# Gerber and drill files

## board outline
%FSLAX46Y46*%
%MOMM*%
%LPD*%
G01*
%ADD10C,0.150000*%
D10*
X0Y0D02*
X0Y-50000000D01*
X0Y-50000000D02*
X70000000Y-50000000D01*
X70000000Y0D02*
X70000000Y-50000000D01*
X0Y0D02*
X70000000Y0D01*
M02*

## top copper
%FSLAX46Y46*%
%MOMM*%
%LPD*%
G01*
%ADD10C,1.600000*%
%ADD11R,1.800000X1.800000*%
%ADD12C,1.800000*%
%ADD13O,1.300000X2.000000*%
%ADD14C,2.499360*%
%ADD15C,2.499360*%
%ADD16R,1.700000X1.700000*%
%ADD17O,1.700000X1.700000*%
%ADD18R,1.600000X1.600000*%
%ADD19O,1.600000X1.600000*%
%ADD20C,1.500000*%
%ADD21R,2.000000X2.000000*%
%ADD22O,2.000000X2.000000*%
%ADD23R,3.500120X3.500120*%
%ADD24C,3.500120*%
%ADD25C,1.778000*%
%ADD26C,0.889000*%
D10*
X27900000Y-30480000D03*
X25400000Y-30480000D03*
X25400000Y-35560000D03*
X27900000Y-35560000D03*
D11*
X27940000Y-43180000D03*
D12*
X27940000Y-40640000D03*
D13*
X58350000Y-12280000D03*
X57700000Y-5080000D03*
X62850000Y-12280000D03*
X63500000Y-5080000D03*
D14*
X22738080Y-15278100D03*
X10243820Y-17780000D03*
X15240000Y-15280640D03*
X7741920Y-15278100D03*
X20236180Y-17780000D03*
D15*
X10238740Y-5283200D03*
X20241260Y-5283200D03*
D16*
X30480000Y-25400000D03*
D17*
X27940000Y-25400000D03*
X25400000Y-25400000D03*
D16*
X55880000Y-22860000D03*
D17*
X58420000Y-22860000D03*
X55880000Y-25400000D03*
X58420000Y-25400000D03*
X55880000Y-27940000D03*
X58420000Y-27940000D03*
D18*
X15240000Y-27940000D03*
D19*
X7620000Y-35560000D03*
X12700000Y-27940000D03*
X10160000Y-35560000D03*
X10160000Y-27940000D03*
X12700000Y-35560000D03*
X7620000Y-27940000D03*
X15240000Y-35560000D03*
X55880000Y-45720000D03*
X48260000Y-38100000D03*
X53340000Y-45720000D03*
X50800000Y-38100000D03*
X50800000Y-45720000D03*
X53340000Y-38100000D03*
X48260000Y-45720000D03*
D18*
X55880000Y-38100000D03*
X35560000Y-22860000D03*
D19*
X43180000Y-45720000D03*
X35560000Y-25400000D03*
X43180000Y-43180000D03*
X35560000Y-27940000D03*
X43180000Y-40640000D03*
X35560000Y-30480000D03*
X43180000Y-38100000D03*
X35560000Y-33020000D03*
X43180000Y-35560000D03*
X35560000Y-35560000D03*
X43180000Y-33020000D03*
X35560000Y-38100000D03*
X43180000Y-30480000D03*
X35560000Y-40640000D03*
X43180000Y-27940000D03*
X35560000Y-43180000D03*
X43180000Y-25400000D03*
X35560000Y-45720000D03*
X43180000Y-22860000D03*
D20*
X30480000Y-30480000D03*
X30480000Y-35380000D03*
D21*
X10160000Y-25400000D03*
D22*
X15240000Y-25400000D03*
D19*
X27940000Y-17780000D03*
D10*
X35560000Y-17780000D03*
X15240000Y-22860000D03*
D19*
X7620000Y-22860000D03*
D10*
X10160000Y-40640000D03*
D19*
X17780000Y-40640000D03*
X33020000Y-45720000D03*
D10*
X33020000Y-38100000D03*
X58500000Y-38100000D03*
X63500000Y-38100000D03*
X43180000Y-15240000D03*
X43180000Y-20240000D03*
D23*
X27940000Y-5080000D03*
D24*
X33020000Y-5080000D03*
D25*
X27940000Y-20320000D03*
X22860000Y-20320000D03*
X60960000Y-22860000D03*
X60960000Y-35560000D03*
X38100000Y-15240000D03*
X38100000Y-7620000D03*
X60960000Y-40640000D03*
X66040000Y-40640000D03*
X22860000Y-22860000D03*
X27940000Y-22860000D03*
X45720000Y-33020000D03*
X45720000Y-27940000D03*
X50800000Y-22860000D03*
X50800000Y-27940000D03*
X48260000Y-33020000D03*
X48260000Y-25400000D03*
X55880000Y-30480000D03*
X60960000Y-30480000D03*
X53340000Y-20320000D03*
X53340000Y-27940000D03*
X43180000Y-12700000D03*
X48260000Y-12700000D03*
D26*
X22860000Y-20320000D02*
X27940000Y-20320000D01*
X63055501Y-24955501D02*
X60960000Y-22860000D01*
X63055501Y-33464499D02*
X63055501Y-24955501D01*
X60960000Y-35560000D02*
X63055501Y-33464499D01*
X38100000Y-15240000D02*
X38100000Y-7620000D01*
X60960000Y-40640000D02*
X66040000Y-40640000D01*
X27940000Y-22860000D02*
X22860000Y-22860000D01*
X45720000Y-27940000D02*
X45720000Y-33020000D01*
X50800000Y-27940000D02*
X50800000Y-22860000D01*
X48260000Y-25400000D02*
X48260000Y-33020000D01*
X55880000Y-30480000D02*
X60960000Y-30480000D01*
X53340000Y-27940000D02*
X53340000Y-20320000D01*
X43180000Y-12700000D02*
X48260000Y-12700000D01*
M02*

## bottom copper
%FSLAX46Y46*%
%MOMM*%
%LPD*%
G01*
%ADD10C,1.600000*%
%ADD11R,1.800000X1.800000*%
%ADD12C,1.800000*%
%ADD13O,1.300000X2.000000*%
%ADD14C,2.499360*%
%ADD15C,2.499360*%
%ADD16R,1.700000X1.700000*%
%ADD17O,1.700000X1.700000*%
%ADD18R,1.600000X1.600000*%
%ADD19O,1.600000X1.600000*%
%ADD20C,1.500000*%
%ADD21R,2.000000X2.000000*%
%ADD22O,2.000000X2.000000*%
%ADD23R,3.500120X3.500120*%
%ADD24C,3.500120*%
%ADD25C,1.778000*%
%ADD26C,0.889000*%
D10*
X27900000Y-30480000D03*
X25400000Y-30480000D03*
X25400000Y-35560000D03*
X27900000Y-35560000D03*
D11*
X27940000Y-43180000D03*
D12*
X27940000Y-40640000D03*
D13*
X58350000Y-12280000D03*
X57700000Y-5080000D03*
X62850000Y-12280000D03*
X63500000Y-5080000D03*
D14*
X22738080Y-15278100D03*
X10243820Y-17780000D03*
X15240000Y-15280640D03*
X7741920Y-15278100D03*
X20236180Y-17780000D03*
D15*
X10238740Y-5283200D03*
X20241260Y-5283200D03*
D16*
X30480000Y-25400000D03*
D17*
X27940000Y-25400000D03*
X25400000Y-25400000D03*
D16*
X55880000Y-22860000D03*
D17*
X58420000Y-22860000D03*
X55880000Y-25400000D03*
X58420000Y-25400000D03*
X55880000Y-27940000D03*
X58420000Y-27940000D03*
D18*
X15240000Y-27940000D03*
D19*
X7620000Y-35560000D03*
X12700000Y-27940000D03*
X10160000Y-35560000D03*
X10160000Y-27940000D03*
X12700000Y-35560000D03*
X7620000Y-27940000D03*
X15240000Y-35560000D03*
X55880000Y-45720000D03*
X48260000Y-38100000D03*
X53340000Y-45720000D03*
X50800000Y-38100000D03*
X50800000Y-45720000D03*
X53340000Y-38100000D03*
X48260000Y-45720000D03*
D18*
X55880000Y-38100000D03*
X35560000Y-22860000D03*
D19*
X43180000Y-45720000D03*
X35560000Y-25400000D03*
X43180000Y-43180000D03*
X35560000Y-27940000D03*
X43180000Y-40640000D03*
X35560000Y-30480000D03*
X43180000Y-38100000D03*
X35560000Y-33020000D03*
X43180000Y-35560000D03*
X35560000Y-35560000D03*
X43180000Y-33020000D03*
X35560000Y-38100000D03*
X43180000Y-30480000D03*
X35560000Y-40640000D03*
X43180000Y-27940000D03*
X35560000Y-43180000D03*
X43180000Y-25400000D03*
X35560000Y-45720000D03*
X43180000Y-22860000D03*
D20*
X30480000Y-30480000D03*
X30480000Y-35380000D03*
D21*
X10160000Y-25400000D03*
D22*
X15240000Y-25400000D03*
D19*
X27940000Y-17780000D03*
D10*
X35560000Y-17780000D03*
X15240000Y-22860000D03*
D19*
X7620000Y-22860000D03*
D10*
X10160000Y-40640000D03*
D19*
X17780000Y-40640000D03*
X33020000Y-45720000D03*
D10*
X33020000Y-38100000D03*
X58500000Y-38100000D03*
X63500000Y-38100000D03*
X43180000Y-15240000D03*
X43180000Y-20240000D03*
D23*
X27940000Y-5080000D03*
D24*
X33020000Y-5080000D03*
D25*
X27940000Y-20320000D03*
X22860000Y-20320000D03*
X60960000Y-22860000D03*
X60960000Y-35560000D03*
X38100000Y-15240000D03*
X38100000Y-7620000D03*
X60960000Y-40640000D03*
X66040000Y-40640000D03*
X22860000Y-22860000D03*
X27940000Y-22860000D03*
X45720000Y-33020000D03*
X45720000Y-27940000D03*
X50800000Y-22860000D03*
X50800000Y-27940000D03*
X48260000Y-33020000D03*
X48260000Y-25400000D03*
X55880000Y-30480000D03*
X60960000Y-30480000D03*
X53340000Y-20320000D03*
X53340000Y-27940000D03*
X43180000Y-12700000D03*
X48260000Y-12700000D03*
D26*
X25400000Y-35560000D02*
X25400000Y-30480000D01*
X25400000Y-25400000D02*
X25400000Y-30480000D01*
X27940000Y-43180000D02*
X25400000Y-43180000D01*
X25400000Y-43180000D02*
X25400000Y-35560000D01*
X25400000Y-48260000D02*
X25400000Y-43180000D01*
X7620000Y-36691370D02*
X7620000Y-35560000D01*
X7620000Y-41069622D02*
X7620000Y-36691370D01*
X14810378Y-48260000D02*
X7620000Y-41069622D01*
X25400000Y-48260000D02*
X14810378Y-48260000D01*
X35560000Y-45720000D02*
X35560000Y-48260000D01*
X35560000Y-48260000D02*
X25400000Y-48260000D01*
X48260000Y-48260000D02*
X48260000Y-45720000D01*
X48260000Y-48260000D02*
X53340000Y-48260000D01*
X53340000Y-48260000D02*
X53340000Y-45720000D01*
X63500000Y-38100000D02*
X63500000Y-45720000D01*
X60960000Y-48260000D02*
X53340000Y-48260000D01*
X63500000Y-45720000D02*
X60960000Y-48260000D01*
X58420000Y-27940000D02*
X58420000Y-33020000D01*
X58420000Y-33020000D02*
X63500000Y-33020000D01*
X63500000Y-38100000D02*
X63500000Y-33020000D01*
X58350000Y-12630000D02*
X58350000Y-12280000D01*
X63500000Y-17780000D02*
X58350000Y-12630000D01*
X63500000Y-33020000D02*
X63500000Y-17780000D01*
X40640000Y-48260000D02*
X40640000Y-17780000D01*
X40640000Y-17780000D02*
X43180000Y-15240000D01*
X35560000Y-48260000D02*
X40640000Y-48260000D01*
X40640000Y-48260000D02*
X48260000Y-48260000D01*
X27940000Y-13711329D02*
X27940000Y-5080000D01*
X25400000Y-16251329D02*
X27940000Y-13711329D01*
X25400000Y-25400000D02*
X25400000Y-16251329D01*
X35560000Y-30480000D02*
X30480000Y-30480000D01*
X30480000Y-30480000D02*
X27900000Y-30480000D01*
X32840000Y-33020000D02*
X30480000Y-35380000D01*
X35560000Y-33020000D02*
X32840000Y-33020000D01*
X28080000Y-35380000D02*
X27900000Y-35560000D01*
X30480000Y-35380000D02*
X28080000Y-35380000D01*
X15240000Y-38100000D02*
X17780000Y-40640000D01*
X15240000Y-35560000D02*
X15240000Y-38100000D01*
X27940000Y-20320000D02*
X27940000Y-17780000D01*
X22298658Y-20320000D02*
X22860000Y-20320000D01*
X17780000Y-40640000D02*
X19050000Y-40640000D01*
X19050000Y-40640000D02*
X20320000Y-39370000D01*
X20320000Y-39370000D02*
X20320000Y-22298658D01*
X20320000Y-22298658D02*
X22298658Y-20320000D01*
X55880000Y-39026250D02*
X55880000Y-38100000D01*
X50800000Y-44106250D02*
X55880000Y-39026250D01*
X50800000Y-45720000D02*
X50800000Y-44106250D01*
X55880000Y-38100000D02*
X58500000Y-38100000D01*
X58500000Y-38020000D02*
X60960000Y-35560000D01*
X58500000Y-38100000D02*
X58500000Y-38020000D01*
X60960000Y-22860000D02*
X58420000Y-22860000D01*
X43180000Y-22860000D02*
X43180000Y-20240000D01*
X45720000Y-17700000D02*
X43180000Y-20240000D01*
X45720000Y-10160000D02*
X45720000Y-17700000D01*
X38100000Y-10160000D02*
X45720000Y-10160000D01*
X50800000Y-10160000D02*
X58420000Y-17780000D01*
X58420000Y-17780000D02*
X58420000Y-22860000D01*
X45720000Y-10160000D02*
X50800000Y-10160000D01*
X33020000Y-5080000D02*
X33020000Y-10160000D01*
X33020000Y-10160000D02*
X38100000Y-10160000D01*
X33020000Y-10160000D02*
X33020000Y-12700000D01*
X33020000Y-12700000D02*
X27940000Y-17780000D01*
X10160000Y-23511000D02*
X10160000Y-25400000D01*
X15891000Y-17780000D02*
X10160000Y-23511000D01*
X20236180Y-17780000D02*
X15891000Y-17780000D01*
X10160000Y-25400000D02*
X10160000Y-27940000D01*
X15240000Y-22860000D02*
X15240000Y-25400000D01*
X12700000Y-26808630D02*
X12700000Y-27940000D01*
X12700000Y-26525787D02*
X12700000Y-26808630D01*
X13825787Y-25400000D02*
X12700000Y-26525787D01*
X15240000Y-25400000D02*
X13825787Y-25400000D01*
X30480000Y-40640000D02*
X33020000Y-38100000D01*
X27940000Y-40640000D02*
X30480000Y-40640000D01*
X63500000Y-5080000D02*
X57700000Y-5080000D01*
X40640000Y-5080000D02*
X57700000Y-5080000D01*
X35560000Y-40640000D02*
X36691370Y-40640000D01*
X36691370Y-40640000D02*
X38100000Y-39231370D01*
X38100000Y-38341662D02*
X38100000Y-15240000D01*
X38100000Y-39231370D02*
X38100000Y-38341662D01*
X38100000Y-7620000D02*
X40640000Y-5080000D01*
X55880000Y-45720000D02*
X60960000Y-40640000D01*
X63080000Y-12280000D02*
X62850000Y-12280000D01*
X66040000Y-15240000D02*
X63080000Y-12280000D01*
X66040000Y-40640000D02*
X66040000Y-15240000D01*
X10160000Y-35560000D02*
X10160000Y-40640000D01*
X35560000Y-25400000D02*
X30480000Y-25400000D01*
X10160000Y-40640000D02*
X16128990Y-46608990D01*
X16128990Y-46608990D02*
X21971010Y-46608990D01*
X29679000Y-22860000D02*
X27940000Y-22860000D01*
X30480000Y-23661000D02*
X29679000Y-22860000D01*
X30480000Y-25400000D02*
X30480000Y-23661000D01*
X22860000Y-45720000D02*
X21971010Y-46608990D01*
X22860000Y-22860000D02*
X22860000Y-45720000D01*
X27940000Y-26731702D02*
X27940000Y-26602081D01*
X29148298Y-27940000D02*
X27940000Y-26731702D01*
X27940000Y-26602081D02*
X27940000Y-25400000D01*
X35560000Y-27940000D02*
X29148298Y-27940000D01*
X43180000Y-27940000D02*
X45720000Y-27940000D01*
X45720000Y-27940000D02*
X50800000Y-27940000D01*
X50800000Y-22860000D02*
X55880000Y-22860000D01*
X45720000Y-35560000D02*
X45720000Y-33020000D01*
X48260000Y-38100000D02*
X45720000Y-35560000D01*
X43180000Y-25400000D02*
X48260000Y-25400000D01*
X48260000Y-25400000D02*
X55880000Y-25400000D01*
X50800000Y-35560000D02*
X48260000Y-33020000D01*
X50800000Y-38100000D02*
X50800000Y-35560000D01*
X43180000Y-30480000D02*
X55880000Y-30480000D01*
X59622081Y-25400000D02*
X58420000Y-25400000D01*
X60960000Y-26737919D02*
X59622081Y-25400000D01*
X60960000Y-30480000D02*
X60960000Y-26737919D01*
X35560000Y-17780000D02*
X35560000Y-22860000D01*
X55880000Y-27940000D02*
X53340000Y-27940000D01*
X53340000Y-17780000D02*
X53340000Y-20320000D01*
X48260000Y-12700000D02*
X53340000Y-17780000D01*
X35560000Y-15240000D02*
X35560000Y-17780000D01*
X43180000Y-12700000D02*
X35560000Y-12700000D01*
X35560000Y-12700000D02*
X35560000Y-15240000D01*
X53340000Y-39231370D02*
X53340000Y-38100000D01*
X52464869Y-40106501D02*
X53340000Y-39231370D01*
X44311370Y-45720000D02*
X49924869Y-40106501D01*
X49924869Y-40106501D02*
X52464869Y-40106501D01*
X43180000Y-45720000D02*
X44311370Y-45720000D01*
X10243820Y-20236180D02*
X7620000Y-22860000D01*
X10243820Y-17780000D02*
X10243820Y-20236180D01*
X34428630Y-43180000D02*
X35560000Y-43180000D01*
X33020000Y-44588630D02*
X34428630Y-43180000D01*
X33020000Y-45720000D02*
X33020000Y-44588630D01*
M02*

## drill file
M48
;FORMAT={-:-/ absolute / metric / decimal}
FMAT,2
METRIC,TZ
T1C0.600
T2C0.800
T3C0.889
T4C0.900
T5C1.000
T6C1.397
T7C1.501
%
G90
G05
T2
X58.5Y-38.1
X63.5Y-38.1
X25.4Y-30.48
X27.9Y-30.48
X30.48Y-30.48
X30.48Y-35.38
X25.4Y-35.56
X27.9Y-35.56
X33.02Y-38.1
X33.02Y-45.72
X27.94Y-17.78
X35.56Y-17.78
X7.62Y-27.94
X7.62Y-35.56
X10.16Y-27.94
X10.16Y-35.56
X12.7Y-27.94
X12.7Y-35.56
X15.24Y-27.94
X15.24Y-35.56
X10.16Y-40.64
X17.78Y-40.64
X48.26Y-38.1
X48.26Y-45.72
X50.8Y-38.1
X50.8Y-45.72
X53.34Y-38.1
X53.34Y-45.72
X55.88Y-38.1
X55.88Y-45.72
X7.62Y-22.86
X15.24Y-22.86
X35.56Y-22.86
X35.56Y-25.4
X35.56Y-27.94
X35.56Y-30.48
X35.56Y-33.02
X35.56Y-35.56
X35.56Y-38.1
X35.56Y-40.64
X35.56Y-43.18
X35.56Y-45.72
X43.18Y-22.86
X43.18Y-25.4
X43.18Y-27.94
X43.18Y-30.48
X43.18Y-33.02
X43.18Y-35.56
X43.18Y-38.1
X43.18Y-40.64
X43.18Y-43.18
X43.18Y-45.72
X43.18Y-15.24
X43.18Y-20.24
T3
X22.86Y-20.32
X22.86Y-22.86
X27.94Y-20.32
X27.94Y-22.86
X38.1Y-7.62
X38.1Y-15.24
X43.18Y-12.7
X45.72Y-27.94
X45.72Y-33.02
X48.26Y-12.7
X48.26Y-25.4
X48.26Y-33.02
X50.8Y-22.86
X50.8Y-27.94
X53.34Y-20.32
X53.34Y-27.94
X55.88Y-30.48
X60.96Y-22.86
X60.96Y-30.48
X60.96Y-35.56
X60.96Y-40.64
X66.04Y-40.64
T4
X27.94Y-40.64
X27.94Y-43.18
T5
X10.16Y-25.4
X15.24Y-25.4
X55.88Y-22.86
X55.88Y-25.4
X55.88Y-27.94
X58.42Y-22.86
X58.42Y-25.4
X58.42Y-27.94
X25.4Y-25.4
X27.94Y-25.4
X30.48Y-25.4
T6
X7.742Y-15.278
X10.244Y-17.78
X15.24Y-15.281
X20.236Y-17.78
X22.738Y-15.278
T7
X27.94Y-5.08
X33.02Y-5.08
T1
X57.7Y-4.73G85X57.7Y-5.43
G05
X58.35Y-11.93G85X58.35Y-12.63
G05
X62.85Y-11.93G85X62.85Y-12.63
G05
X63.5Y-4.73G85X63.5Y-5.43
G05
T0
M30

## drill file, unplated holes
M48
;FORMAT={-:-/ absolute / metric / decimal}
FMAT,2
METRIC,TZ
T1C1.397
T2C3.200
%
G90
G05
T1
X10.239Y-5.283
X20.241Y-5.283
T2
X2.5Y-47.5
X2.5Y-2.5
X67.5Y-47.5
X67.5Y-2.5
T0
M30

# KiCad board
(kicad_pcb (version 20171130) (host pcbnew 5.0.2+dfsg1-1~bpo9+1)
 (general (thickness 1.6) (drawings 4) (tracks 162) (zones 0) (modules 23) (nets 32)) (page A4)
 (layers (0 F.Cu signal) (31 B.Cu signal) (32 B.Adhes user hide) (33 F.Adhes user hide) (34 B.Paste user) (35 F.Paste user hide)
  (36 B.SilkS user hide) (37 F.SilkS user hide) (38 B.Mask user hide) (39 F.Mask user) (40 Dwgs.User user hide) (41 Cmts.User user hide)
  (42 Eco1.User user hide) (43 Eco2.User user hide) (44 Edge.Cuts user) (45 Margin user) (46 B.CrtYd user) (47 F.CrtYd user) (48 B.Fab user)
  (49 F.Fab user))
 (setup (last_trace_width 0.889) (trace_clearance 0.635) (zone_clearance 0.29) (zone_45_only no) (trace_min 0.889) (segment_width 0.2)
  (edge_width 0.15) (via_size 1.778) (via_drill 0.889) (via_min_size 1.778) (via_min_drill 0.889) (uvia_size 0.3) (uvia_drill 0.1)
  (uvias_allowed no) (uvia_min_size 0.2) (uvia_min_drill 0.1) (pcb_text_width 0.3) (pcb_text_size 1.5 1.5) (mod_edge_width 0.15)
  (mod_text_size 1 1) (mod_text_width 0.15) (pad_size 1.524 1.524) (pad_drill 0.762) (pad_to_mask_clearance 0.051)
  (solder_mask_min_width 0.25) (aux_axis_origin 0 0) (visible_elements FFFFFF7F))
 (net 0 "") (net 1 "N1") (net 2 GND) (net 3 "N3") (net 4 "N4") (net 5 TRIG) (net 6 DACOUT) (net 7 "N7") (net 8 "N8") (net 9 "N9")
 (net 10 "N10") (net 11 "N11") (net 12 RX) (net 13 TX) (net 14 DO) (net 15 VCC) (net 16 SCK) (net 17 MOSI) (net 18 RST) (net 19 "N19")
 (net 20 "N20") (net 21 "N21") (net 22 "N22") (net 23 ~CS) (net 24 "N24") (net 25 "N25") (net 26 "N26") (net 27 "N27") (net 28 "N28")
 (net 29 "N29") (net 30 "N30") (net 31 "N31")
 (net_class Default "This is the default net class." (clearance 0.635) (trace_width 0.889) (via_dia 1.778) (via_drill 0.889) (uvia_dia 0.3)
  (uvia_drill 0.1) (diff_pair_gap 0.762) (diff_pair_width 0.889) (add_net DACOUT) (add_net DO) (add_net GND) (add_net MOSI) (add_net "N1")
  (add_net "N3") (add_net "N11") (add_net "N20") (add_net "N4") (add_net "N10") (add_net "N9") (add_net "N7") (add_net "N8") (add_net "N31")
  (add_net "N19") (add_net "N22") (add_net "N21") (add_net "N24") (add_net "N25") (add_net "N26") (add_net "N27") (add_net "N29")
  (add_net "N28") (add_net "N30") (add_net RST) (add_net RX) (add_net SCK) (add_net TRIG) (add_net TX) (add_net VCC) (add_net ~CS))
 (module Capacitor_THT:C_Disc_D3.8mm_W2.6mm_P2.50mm (layer F.Cu) (at 27.9 30.48 180)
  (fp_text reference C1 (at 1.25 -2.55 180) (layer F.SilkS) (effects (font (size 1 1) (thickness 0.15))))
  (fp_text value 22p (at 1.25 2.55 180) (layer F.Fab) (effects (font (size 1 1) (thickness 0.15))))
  (pad 1 thru_hole circle (at 0 0 180) (size 1.6 1.6) (drill 0.8) (layers *.Cu *.Mask) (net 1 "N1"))
  (pad 2 thru_hole circle (at 2.5 0 180) (size 1.6 1.6) (drill 0.8) (layers *.Cu *.Mask) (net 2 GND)))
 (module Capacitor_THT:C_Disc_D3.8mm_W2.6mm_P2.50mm (layer F.Cu) (at 27.9 35.56 180)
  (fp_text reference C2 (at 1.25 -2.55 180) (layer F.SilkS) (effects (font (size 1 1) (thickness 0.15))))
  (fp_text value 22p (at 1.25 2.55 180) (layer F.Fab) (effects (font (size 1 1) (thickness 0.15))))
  (pad 2 thru_hole circle (at 2.5 0 180) (size 1.6 1.6) (drill 0.8) (layers *.Cu *.Mask) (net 2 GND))
  (pad 1 thru_hole circle (at 0 0 180) (size 1.6 1.6) (drill 0.8) (layers *.Cu *.Mask) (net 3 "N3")))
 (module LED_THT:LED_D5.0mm (layer F.Cu) (at 27.94 43.18 90)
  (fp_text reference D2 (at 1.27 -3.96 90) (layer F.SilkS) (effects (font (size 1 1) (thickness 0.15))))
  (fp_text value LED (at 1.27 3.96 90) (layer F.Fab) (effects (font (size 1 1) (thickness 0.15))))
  (pad 1 thru_hole rect (at 0 0 90) (size 1.8 1.8) (drill 0.9) (layers *.Cu *.Mask) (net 2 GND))
  (pad 2 thru_hole circle (at 2.54 0 90) (size 1.8 1.8) (drill 0.9) (layers *.Cu *.Mask) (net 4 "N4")))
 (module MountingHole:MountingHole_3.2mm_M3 (layer F.Cu) (at 2.5 2.5)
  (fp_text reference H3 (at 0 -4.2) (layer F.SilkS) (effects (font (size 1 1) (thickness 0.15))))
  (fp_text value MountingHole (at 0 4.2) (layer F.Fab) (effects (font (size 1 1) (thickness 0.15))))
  (pad 1 np_thru_hole circle (at 0 0) (size 3.2 3.2) (drill 3.2) (layers *.Cu *.Mask)))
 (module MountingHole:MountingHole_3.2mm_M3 (layer F.Cu) (at 67.5 2.5)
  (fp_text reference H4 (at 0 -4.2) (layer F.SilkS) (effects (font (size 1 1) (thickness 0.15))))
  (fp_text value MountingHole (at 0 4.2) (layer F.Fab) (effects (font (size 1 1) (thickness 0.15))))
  (pad 1 np_thru_hole circle (at 0 0) (size 3.2 3.2) (drill 3.2) (layers *.Cu *.Mask)))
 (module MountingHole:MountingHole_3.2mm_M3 (layer F.Cu) (at 67.5 47.5)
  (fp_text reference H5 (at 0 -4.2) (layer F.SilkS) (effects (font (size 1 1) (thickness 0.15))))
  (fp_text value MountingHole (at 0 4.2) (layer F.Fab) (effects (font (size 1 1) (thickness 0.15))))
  (pad 1 np_thru_hole circle (at 0 0) (size 3.2 3.2) (drill 3.2) (layers *.Cu *.Mask)))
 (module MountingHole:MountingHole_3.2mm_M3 (layer F.Cu) (at 2.5 47.5)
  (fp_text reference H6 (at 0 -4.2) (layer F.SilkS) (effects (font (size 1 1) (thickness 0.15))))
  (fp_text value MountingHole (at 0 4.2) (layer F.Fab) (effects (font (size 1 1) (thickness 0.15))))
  (pad 1 np_thru_hole circle (at 0 0) (size 3.2 3.2) (drill 3.2) (layers *.Cu *.Mask)))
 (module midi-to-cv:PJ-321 (layer F.Cu) (at 60.6 8.68)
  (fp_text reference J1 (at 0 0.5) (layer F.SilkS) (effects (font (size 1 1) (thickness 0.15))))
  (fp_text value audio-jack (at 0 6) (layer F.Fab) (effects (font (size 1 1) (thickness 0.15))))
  (pad 1 thru_hole oval (at -2.25 3.6) (size 1.3 2) (drill oval 0.6 1.3) (layers *.Cu *.Mask) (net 2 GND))
  (pad 2 thru_hole oval (at -2.9 -3.6) (size 1.3 2) (drill oval 0.6 1.3) (layers *.Cu *.Mask) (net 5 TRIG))
  (pad 3 thru_hole oval (at 2.25 3.6) (size 1.3 2) (drill oval 0.6 1.3) (layers *.Cu *.Mask) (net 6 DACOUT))
  (pad 2 thru_hole oval (at 2.9 -3.6) (size 1.3 2) (drill oval 0.6 1.3) (layers *.Cu *.Mask) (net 5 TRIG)))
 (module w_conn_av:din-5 (layer F.Cu) (at 15.24 12.2809 180)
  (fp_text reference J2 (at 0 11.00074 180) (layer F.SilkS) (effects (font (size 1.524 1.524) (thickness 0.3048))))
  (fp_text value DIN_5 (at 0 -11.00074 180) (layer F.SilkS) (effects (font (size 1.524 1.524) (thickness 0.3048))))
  (pad 3 thru_hole circle (at -7.49808 -2.9972 180) (size 2.49936 2.49936) (drill 1.397) (layers *.Cu *.SilkS *.Mask) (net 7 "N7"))
  (pad 4 thru_hole circle (at 4.99618 -5.4991 180) (size 2.49936 2.49936) (drill 1.397) (layers *.Cu *.SilkS *.Mask) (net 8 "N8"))
  (pad 2 thru_hole circle (at 0 -2.99974 180) (size 2.49936 2.49936) (drill 1.397) (layers *.Cu *.SilkS *.Mask) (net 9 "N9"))
  (pad 1 thru_hole circle (at 7.49808 -2.9972 180) (size 2.49936 2.49936) (drill 1.397) (layers *.Cu *.SilkS *.Mask) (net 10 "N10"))
  (pad 5 thru_hole circle (at -4.99618 -5.4991 180) (size 2.49936 2.49936) (drill 1.397) (layers *.Cu *.SilkS *.Mask) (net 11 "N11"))
  (pad "" np_thru_hole circle (at 5.00126 6.9977 180) (size 2.49936 2.49936) (drill 1.397) (layers *.Cu *.Mask F.SilkS))
  (pad "" np_thru_hole circle (at -5.00126 6.9977 180) (size 2.49936 2.49936) (drill 1.397) (layers *.Cu *.Mask F.SilkS)))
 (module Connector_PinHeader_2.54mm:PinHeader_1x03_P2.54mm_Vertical (layer F.Cu) (at 30.48 25.4 270)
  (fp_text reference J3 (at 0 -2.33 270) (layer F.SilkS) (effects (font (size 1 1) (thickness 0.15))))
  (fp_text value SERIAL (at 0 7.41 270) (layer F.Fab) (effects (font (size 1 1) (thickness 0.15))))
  (pad 1 thru_hole rect (at 0 0 270) (size 1.7 1.7) (drill 1) (layers *.Cu *.Mask) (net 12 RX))
  (pad 2 thru_hole oval (at 0 2.54 270) (size 1.7 1.7) (drill 1) (layers *.Cu *.Mask) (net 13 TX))
  (pad 3 thru_hole oval (at 0 5.08 270) (size 1.7 1.7) (drill 1) (layers *.Cu *.Mask) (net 2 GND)))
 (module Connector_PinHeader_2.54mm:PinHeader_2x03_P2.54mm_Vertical (layer F.Cu) (at 55.88 22.86)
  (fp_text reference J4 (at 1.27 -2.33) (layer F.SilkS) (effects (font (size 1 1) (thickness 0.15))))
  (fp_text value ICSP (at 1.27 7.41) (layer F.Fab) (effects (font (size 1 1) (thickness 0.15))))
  (pad 1 thru_hole rect (at 0 0) (size 1.7 1.7) (drill 1) (layers *.Cu *.Mask) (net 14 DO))
  (pad 2 thru_hole oval (at 2.54 0) (size 1.7 1.7) (drill 1) (layers *.Cu *.Mask) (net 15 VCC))
  (pad 3 thru_hole oval (at 0 2.54) (size 1.7 1.7) (drill 1) (layers *.Cu *.Mask) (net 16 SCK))
  (pad 4 thru_hole oval (at 2.54 2.54) (size 1.7 1.7) (drill 1) (layers *.Cu *.Mask) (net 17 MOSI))
  (pad 5 thru_hole oval (at 0 5.08) (size 1.7 1.7) (drill 1) (layers *.Cu *.Mask) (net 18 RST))
  (pad 6 thru_hole oval (at 2.54 5.08) (size 1.7 1.7) (drill 1) (layers *.Cu *.Mask) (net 2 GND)))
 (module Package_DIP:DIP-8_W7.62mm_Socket (layer F.Cu) (at 15.24 27.94 270)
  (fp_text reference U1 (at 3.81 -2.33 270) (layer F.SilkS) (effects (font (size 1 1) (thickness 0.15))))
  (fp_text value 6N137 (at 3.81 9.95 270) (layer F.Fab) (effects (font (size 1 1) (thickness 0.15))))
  (pad 1 thru_hole rect (at 0 0 270) (size 1.6 1.6) (drill 0.8) (layers *.Cu *.Mask) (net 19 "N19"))
  (pad 5 thru_hole oval (at 7.62 7.62 270) (size 1.6 1.6) (drill 0.8) (layers *.Cu *.Mask) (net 2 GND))
  (pad 2 thru_hole oval (at 0 2.54 270) (size 1.6 1.6) (drill 0.8) (layers *.Cu *.Mask) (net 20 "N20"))
  (pad 6 thru_hole oval (at 7.62 5.08 270) (size 1.6 1.6) (drill 0.8) (layers *.Cu *.Mask) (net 12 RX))
  (pad 3 thru_hole oval (at 0 5.08 270) (size 1.6 1.6) (drill 0.8) (layers *.Cu *.Mask) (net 11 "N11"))
  (pad 7 thru_hole oval (at 7.62 2.54 270) (size 1.6 1.6) (drill 0.8) (layers *.Cu *.Mask) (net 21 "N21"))
  (pad 4 thru_hole oval (at 0 7.62 270) (size 1.6 1.6) (drill 0.8) (layers *.Cu *.Mask) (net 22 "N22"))
  (pad 8 thru_hole oval (at 7.62 0 270) (size 1.6 1.6) (drill 0.8) (layers *.Cu *.Mask) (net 15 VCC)))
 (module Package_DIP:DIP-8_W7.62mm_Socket (layer F.Cu) (at 55.88 38.1 270)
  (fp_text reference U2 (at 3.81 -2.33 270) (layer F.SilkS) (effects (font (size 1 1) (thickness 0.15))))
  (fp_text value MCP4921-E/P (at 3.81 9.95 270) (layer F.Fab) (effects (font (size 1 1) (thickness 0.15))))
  (pad 8 thru_hole oval (at 7.62 0 270) (size 1.6 1.6) (drill 0.8) (layers *.Cu *.Mask) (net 6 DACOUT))
  (pad 4 thru_hole oval (at 0 7.62 270) (size 1.6 1.6) (drill 0.8) (layers *.Cu *.Mask) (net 14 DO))
  (pad 7 thru_hole oval (at 7.62 2.54 270) (size 1.6 1.6) (drill 0.8) (layers *.Cu *.Mask) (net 2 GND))
  (pad 3 thru_hole oval (at 0 5.08 270) (size 1.6 1.6) (drill 0.8) (layers *.Cu *.Mask) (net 16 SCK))
  (pad 6 thru_hole oval (at 7.62 5.08 270) (size 1.6 1.6) (drill 0.8) (layers *.Cu *.Mask) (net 15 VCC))
  (pad 2 thru_hole oval (at 0 2.54 270) (size 1.6 1.6) (drill 0.8) (layers *.Cu *.Mask) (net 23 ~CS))
  (pad 5 thru_hole oval (at 7.62 7.62 270) (size 1.6 1.6) (drill 0.8) (layers *.Cu *.Mask) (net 2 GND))
  (pad 1 thru_hole rect (at 0 0 270) (size 1.6 1.6) (drill 0.8) (layers *.Cu *.Mask) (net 15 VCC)))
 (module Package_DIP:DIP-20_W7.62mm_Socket (layer F.Cu) (at 35.56 22.86)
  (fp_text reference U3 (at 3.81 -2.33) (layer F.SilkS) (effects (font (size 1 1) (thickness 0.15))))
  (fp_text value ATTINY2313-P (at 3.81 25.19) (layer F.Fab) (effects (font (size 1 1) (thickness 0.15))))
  (pad 1 thru_hole rect (at 0 0) (size 1.6 1.6) (drill 0.8) (layers *.Cu *.Mask) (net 18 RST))
  (pad 11 thru_hole oval (at 7.62 22.86) (size 1.6 1.6) (drill 0.8) (layers *.Cu *.Mask) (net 23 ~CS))
  (pad 2 thru_hole oval (at 0 2.54) (size 1.6 1.6) (drill 0.8) (layers *.Cu *.Mask) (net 12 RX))
  (pad 12 thru_hole oval (at 7.62 20.32) (size 1.6 1.6) (drill 0.8) (layers *.Cu *.Mask) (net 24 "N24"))
  (pad 3 thru_hole oval (at 0 5.08) (size 1.6 1.6) (drill 0.8) (layers *.Cu *.Mask) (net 13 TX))
  (pad 13 thru_hole oval (at 7.62 17.78) (size 1.6 1.6) (drill 0.8) (layers *.Cu *.Mask) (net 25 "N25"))
  (pad 4 thru_hole oval (at 0 7.62) (size 1.6 1.6) (drill 0.8) (layers *.Cu *.Mask) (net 1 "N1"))
  (pad 14 thru_hole oval (at 7.62 15.24) (size 1.6 1.6) (drill 0.8) (layers *.Cu *.Mask) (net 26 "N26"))
  (pad 5 thru_hole oval (at 0 10.16) (size 1.6 1.6) (drill 0.8) (layers *.Cu *.Mask) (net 3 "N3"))
  (pad 15 thru_hole oval (at 7.62 12.7) (size 1.6 1.6) (drill 0.8) (layers *.Cu *.Mask) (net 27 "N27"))
  (pad 6 thru_hole oval (at 0 12.7) (size 1.6 1.6) (drill 0.8) (layers *.Cu *.Mask) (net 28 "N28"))
  (pad 16 thru_hole oval (at 7.62 10.16) (size 1.6 1.6) (drill 0.8) (layers *.Cu *.Mask) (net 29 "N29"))
  (pad 7 thru_hole oval (at 0 15.24) (size 1.6 1.6) (drill 0.8) (layers *.Cu *.Mask) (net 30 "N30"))
  (pad 17 thru_hole oval (at 7.62 7.62) (size 1.6 1.6) (drill 0.8) (layers *.Cu *.Mask) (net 17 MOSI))
  (pad 8 thru_hole oval (at 0 17.78) (size 1.6 1.6) (drill 0.8) (layers *.Cu *.Mask) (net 5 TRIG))
  (pad 18 thru_hole oval (at 7.62 5.08) (size 1.6 1.6) (drill 0.8) (layers *.Cu *.Mask) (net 14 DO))
  (pad 9 thru_hole oval (at 0 20.32) (size 1.6 1.6) (drill 0.8) (layers *.Cu *.Mask) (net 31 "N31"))
  (pad 19 thru_hole oval (at 7.62 2.54) (size 1.6 1.6) (drill 0.8) (layers *.Cu *.Mask) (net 16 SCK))
  (pad 10 thru_hole oval (at 0 22.86) (size 1.6 1.6) (drill 0.8) (layers *.Cu *.Mask) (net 2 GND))
  (pad 20 thru_hole oval (at 7.62 0) (size 1.6 1.6) (drill 0.8) (layers *.Cu *.Mask) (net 15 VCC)))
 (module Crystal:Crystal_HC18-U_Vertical (layer F.Cu) (at 30.48 30.48 270)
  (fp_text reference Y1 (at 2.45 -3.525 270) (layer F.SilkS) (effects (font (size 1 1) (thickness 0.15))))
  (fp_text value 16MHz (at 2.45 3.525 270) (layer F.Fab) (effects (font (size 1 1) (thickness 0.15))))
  (pad 1 thru_hole circle (at 0 0 270) (size 1.5 1.5) (drill 0.8) (layers *.Cu *.Mask) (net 1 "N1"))
  (pad 2 thru_hole circle (at 4.9 0 270) (size 1.5 1.5) (drill 0.8) (layers *.Cu *.Mask) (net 3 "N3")))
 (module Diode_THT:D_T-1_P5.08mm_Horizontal (layer F.Cu) (at 10.16 25.4)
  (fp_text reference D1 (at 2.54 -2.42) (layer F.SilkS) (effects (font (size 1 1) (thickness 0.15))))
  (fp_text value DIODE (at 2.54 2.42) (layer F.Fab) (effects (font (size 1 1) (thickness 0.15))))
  (pad 1 thru_hole rect (at 0 0) (size 2 2) (drill 1) (layers *.Cu *.Mask) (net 11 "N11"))
  (pad 2 thru_hole oval (at 5.08 0) (size 2 2) (drill 1) (layers *.Cu *.Mask) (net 20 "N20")))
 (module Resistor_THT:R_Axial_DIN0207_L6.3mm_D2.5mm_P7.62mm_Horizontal (layer F.Cu) (at 35.56 17.78 180)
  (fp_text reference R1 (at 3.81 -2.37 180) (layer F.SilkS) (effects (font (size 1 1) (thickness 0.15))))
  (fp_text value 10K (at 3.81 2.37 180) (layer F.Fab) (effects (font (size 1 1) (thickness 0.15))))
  (pad 2 thru_hole oval (at 7.62 0 180) (size 1.6 1.6) (drill 0.8) (layers *.Cu *.Mask) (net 15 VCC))
  (pad 1 thru_hole circle (at 0 0 180) (size 1.6 1.6) (drill 0.8) (layers *.Cu *.Mask) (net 18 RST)))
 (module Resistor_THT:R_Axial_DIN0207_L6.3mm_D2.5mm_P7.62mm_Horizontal (layer F.Cu) (at 15.24 22.86 180)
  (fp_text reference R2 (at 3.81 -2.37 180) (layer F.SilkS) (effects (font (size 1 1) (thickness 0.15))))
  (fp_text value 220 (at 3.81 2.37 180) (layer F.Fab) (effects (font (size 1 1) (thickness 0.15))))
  (pad 1 thru_hole circle (at 0 0 180) (size 1.6 1.6) (drill 0.8) (layers *.Cu *.Mask) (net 20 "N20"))
  (pad 2 thru_hole oval (at 7.62 0 180) (size 1.6 1.6) (drill 0.8) (layers *.Cu *.Mask) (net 8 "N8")))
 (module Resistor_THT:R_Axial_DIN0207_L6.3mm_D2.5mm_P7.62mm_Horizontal (layer F.Cu) (at 10.16 40.64)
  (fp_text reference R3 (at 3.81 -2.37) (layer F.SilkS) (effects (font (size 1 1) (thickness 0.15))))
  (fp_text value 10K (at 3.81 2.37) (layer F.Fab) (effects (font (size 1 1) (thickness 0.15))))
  (pad 1 thru_hole circle (at 0 0) (size 1.6 1.6) (drill 0.8) (layers *.Cu *.Mask) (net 12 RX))
  (pad 2 thru_hole oval (at 7.62 0) (size 1.6 1.6) (drill 0.8) (layers *.Cu *.Mask) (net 15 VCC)))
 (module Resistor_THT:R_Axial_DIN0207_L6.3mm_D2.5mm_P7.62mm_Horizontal (layer F.Cu) (at 33.02 38.1 270)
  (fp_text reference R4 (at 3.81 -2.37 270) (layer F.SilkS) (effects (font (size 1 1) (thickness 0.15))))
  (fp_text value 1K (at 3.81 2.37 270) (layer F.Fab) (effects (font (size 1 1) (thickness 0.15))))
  (pad 2 thru_hole oval (at 7.62 0 270) (size 1.6 1.6) (drill 0.8) (layers *.Cu *.Mask) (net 31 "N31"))
  (pad 1 thru_hole circle (at 0 0 270) (size 1.6 1.6) (drill 0.8) (layers *.Cu *.Mask) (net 4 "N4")))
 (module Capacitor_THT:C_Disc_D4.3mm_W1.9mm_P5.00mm (layer F.Cu) (at 58.5 38.1)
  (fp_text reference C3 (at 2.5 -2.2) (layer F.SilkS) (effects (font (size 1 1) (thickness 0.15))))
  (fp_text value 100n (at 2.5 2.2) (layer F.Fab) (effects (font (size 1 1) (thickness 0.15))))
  (pad 1 thru_hole circle (at 0 0) (size 1.6 1.6) (drill 0.8) (layers *.Cu *.Mask) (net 15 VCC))
  (pad 2 thru_hole circle (at 5 0) (size 1.6 1.6) (drill 0.8) (layers *.Cu *.Mask) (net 2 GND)))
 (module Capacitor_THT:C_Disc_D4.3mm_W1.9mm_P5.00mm (layer F.Cu) (at 43.18 20.24 90)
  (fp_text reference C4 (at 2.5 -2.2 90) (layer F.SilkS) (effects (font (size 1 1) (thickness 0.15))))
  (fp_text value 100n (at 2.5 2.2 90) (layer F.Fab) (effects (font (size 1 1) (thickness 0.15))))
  (pad 2 thru_hole circle (at 5 0 90) (size 1.6 1.6) (drill 0.8) (layers *.Cu *.Mask) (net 2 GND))
  (pad 1 thru_hole circle (at 0 0 90) (size 1.6 1.6) (drill 0.8) (layers *.Cu *.Mask) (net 15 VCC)))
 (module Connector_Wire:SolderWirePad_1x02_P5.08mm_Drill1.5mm (layer F.Cu) (at 27.94 5.08)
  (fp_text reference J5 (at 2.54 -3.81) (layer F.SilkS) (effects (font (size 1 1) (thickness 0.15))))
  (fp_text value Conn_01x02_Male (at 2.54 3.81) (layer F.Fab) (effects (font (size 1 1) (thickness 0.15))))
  (pad 1 thru_hole rect (at 0 0) (size 3.50012 3.50012) (drill 1.50114) (layers *.Cu *.Mask) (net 2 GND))
  (pad 2 thru_hole circle (at 5.08 0) (size 3.50012 3.50012) (drill 1.50114) (layers *.Cu *.Mask) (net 15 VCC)))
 (gr_line (start 0 0) (end 0 50) (layer Edge.Cuts) (width 0.15))
 (gr_line (start 0 50) (end 70 50) (layer Edge.Cuts) (width 0.15))
 (gr_line (start 70 0) (end 70 50) (layer Edge.Cuts) (width 0.15))
 (gr_line (start 0 0) (end 70 0) (layer Edge.Cuts) (width 0.15))
 (segment (start 25.4 35.56) (end 25.4 30.48) (width 0.889) (layer B.Cu) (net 2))
 (segment (start 25.4 25.4) (end 25.4 30.48) (width 0.889) (layer B.Cu) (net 2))
 (segment (start 27.94 43.18) (end 25.4 43.18) (width 0.889) (layer B.Cu) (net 2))
 (segment (start 25.4 43.18) (end 25.4 35.56) (width 0.889) (layer B.Cu) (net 2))
 (segment (start 25.4 48.26) (end 25.4 43.18) (width 0.889) (layer B.Cu) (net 2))
 (segment (start 7.62 36.69137) (end 7.62 35.56) (width 0.889) (layer B.Cu) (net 2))
 (segment (start 7.62 41.069622) (end 7.62 36.69137) (width 0.889) (layer B.Cu) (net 2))
 (segment (start 14.810378 48.26) (end 7.62 41.069622) (width 0.889) (layer B.Cu) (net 2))
 (segment (start 25.4 48.26) (end 14.810378 48.26) (width 0.889) (layer B.Cu) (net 2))
 (segment (start 35.56 45.72) (end 35.56 48.26) (width 0.889) (layer B.Cu) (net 2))
 (segment (start 35.56 48.26) (end 25.4 48.26) (width 0.889) (layer B.Cu) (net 2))
 (segment (start 48.26 48.26) (end 48.26 45.72) (width 0.889) (layer B.Cu) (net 2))
 (segment (start 48.26 48.26) (end 53.34 48.26) (width 0.889) (layer B.Cu) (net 2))
 (segment (start 53.34 48.26) (end 53.34 45.72) (width 0.889) (layer B.Cu) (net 2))
 (segment (start 63.5 38.1) (end 63.5 45.72) (width 0.889) (layer B.Cu) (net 2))
 (segment (start 60.96 48.26) (end 53.34 48.26) (width 0.889) (layer B.Cu) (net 2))
 (segment (start 63.5 45.72) (end 60.96 48.26) (width 0.889) (layer B.Cu) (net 2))
 (segment (start 58.42 27.94) (end 58.42 33.02) (width 0.889) (layer B.Cu) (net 2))
 (segment (start 58.42 33.02) (end 63.5 33.02) (width 0.889) (layer B.Cu) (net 2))
 (segment (start 63.5 38.1) (end 63.5 33.02) (width 0.889) (layer B.Cu) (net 2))
 (segment (start 58.35 12.63) (end 58.35 12.28) (width 0.889) (layer B.Cu) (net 2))
 (segment (start 63.5 17.78) (end 58.35 12.63) (width 0.889) (layer B.Cu) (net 2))
 (segment (start 63.5 33.02) (end 63.5 17.78) (width 0.889) (layer B.Cu) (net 2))
 (segment (start 40.64 48.26) (end 40.64 17.78) (width 0.889) (layer B.Cu) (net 2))
 (segment (start 40.64 17.78) (end 43.18 15.24) (width 0.889) (layer B.Cu) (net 2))
 (segment (start 35.56 48.26) (end 40.64 48.26) (width 0.889) (layer B.Cu) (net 2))
 (segment (start 40.64 48.26) (end 48.26 48.26) (width 0.889) (layer B.Cu) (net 2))
 (segment (start 27.94 13.711329) (end 27.94 5.08) (width 0.889) (layer B.Cu) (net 2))
 (segment (start 25.4 16.251329) (end 27.94 13.711329) (width 0.889) (layer B.Cu) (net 2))
 (segment (start 25.4 25.4) (end 25.4 16.251329) (width 0.889) (layer B.Cu) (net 2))
 (segment (start 35.56 30.48) (end 30.48 30.48) (width 0.889) (layer B.Cu) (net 1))
 (segment (start 30.48 30.48) (end 27.9 30.48) (width 0.889) (layer B.Cu) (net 1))
 (segment (start 32.84 33.02) (end 30.48 35.38) (width 0.889) (layer B.Cu) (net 3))
 (segment (start 35.56 33.02) (end 32.84 33.02) (width 0.889) (layer B.Cu) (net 3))
 (segment (start 28.08 35.38) (end 27.9 35.56) (width 0.889) (layer B.Cu) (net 3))
 (segment (start 30.48 35.38) (end 28.08 35.38) (width 0.889) (layer B.Cu) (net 3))
 (segment (start 15.24 38.1) (end 17.78 40.64) (width 0.889) (layer B.Cu) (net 15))
 (segment (start 15.24 35.56) (end 15.24 38.1) (width 0.889) (layer B.Cu) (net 15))
 (segment (start 22.86 20.32) (end 27.94 20.32) (width 0.889) (layer F.Cu) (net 15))
 (segment (start 27.94 20.32) (end 27.94 17.78) (width 0.889) (layer B.Cu) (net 15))
 (segment (start 22.298658 20.32) (end 22.86 20.32) (width 0.889) (layer B.Cu) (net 15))
 (segment (start 17.78 40.64) (end 19.05 40.64) (width 0.889) (layer B.Cu) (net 15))
 (segment (start 19.05 40.64) (end 20.32 39.37) (width 0.889) (layer B.Cu) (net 15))
 (segment (start 20.32 39.37) (end 20.32 22.298658) (width 0.889) (layer B.Cu) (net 15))
 (segment (start 20.32 22.298658) (end 22.298658 20.32) (width 0.889) (layer B.Cu) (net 15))
 (segment (start 55.88 39.02625) (end 55.88 38.1) (width 0.889) (layer B.Cu) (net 15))
 (segment (start 50.8 44.10625) (end 55.88 39.02625) (width 0.889) (layer B.Cu) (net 15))
 (segment (start 50.8 45.72) (end 50.8 44.10625) (width 0.889) (layer B.Cu) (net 15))
 (segment (start 55.88 38.1) (end 58.5 38.1) (width 0.889) (layer B.Cu) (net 15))
 (segment (start 58.5 38.02) (end 60.96 35.56) (width 0.889) (layer B.Cu) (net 15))
 (segment (start 58.5 38.1) (end 58.5 38.02) (width 0.889) (layer B.Cu) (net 15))
 (segment (start 63.055501 24.955501) (end 60.96 22.86) (width 0.889) (layer F.Cu) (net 15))
 (segment (start 63.055501 33.464499) (end 63.055501 24.955501) (width 0.889) (layer F.Cu) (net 15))
 (segment (start 60.96 35.56) (end 63.055501 33.464499) (width 0.889) (layer F.Cu) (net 15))
 (segment (start 60.96 22.86) (end 58.42 22.86) (width 0.889) (layer B.Cu) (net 15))
 (segment (start 43.18 22.86) (end 43.18 20.24) (width 0.889) (layer B.Cu) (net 15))
 (segment (start 45.72 17.7) (end 43.18 20.24) (width 0.889) (layer B.Cu) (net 15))
 (segment (start 45.72 10.16) (end 45.72 17.7) (width 0.889) (layer B.Cu) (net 15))
 (segment (start 38.1 10.16) (end 45.72 10.16) (width 0.889) (layer B.Cu) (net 15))
 (segment (start 50.8 10.16) (end 58.42 17.78) (width 0.889) (layer B.Cu) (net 15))
 (segment (start 58.42 17.78) (end 58.42 22.86) (width 0.889) (layer B.Cu) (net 15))
 (segment (start 45.72 10.16) (end 50.8 10.16) (width 0.889) (layer B.Cu) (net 15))
 (segment (start 33.02 5.08) (end 33.02 10.16) (width 0.889) (layer B.Cu) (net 15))
 (segment (start 33.02 10.16) (end 38.1 10.16) (width 0.889) (layer B.Cu) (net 15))
 (segment (start 33.02 10.16) (end 33.02 12.7) (width 0.889) (layer B.Cu) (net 15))
 (segment (start 33.02 12.7) (end 27.94 17.78) (width 0.889) (layer B.Cu) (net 15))
 (via (at 27.94 20.32) (size 1.778) (drill 0.889) (layers F.Cu B.Cu) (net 15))
 (via (at 22.86 20.32) (size 1.778) (drill 0.889) (layers F.Cu B.Cu) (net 15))
 (via (at 60.96 22.86) (size 1.778) (drill 0.889) (layers F.Cu B.Cu) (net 15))
 (via (at 60.96 35.56) (size 1.778) (drill 0.889) (layers F.Cu B.Cu) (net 15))
 (segment (start 10.16 23.511) (end 10.16 25.4) (width 0.889) (layer B.Cu) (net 11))
 (segment (start 15.891 17.78) (end 10.16 23.511) (width 0.889) (layer B.Cu) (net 11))
 (segment (start 20.23618 17.78) (end 15.891 17.78) (width 0.889) (layer B.Cu) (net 11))
 (segment (start 10.16 25.4) (end 10.16 27.94) (width 0.889) (layer B.Cu) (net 11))
 (segment (start 15.24 22.86) (end 15.24 25.4) (width 0.889) (layer B.Cu) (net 20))
 (segment (start 12.7 26.80863) (end 12.7 27.94) (width 0.889) (layer B.Cu) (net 20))
 (segment (start 12.7 26.525787) (end 12.7 26.80863) (width 0.889) (layer B.Cu) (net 20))
 (segment (start 13.825787 25.4) (end 12.7 26.525787) (width 0.889) (layer B.Cu) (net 20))
 (segment (start 15.24 25.4) (end 13.825787 25.4) (width 0.889) (layer B.Cu) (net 20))
 (segment (start 30.48 40.64) (end 33.02 38.1) (width 0.889) (layer B.Cu) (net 4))
 (segment (start 27.94 40.64) (end 30.48 40.64) (width 0.889) (layer B.Cu) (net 4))
 (segment (start 63.5 5.08) (end 57.7 5.08) (width 0.889) (layer B.Cu) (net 5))
 (segment (start 40.64 5.08) (end 57.7 5.08) (width 0.889) (layer B.Cu) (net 5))
 (segment (start 35.56 40.64) (end 36.69137 40.64) (width 0.889) (layer B.Cu) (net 5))
 (segment (start 36.69137 40.64) (end 38.1 39.23137) (width 0.889) (layer B.Cu) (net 5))
 (via (at 38.1 15.24) (size 1.778) (drill 0.889) (layers F.Cu B.Cu) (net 5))
 (segment (start 38.1 38.341662) (end 38.1 15.24) (width 0.889) (layer B.Cu) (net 5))
 (segment (start 38.1 39.23137) (end 38.1 38.341662) (width 0.889) (layer B.Cu) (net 5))
 (via (at 38.1 7.62) (size 1.778) (drill 0.889) (layers F.Cu B.Cu) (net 5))
 (segment (start 38.1 15.24) (end 38.1 7.62) (width 0.889) (layer F.Cu) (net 5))
 (segment (start 38.1 7.62) (end 40.64 5.08) (width 0.889) (layer B.Cu) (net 5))
 (segment (start 60.96 40.64) (end 66.04 40.64) (width 0.889) (layer F.Cu) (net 6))
 (segment (start 55.88 45.72) (end 60.96 40.64) (width 0.889) (layer B.Cu) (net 6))
 (segment (start 63.08 12.28) (end 62.85 12.28) (width 0.889) (layer B.Cu) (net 6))
 (segment (start 66.04 15.24) (end 63.08 12.28) (width 0.889) (layer B.Cu) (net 6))
 (segment (start 66.04 40.64) (end 66.04 15.24) (width 0.889) (layer B.Cu) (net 6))
 (via (at 60.96 40.64) (size 1.778) (drill 0.889) (layers F.Cu B.Cu) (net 6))
 (via (at 66.04 40.64) (size 1.778) (drill 0.889) (layers F.Cu B.Cu) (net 6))
 (segment (start 10.16 35.56) (end 10.16 40.64) (width 0.889) (layer B.Cu) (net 12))
 (segment (start 35.56 25.4) (end 30.48 25.4) (width 0.889) (layer B.Cu) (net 12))
 (segment (start 10.16 40.64) (end 16.12899 46.60899) (width 0.889) (layer B.Cu) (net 12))
 (segment (start 16.12899 46.60899) (end 21.97101 46.60899) (width 0.889) (layer B.Cu) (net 12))
 (segment (start 29.679 22.86) (end 27.94 22.86) (width 0.889) (layer B.Cu) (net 12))
 (segment (start 30.48 23.661) (end 29.679 22.86) (width 0.889) (layer B.Cu) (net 12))
 (segment (start 30.48 25.4) (end 30.48 23.661) (width 0.889) (layer B.Cu) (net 12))
 (segment (start 27.94 22.86) (end 22.86 22.86) (width 0.889) (layer F.Cu) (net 12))
 (segment (start 22.86 45.72) (end 21.97101 46.60899) (width 0.889) (layer B.Cu) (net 12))
 (segment (start 22.86 22.86) (end 22.86 45.72) (width 0.889) (layer B.Cu) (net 12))
 (via (at 22.86 22.86) (size 1.778) (drill 0.889) (layers F.Cu B.Cu) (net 12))
 (via (at 27.94 22.86) (size 1.778) (drill 0.889) (layers F.Cu B.Cu) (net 12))
 (segment (start 27.94 26.731702) (end 27.94 26.602081) (width 0.889) (layer B.Cu) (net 13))
 (segment (start 29.148298 27.94) (end 27.94 26.731702) (width 0.889) (layer B.Cu) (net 13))
 (segment (start 27.94 26.602081) (end 27.94 25.4) (width 0.889) (layer B.Cu) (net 13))
 (segment (start 35.56 27.94) (end 29.148298 27.94) (width 0.889) (layer B.Cu) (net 13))
 (segment (start 43.18 27.94) (end 45.72 27.94) (width 0.889) (layer B.Cu) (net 14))
 (segment (start 45.72 27.94) (end 45.72 33.02) (width 0.889) (layer F.Cu) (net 14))
 (segment (start 45.72 27.94) (end 50.8 27.94) (width 0.889) (layer B.Cu) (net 14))
 (segment (start 50.8 27.94) (end 50.8 22.86) (width 0.889) (layer F.Cu) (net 14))
 (segment (start 50.8 22.86) (end 55.88 22.86) (width 0.889) (layer B.Cu) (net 14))
 (segment (start 45.72 35.56) (end 45.72 33.02) (width 0.889) (layer B.Cu) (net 14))
 (segment (start 48.26 38.1) (end 45.72 35.56) (width 0.889) (layer B.Cu) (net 14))
 (via (at 45.72 33.02) (size 1.778) (drill 0.889) (layers F.Cu B.Cu) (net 14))
 (via (at 45.72 27.94) (size 1.778) (drill 0.889) (layers F.Cu B.Cu) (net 14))
 (via (at 50.8 22.86) (size 1.778) (drill 0.889) (layers F.Cu B.Cu) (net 14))
 (via (at 50.8 27.94) (size 1.778) (drill 0.889) (layers F.Cu B.Cu) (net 14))
 (segment (start 43.18 25.4) (end 48.26 25.4) (width 0.889) (layer B.Cu) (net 16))
 (segment (start 48.26 25.4) (end 48.26 33.02) (width 0.889) (layer F.Cu) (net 16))
 (segment (start 48.26 25.4) (end 55.88 25.4) (width 0.889) (layer B.Cu) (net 16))
 (segment (start 50.8 35.56) (end 48.26 33.02) (width 0.889) (layer B.Cu) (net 16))
 (segment (start 50.8 38.1) (end 50.8 35.56) (width 0.889) (layer B.Cu) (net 16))
 (via (at 48.26 33.02) (size 1.778) (drill 0.889) (layers F.Cu B.Cu) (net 16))
 (via (at 48.26 25.4) (size 1.778) (drill 0.889) (layers F.Cu B.Cu) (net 16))
 (segment (start 43.18 30.48) (end 55.88 30.48) (width 0.889) (layer B.Cu) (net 17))
 (segment (start 55.88 30.48) (end 60.96 30.48) (width 0.889) (layer F.Cu) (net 17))
 (segment (start 59.622081 25.4) (end 58.42 25.4) (width 0.889) (layer B.Cu) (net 17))
 (segment (start 60.96 26.737919) (end 59.622081 25.4) (width 0.889) (layer B.Cu) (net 17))
 (segment (start 60.96 30.48) (end 60.96 26.737919) (width 0.889) (layer B.Cu) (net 17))
 (via (at 55.88 30.48) (size 1.778) (drill 0.889) (layers F.Cu B.Cu) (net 17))
 (via (at 60.96 30.48) (size 1.778) (drill 0.889) (layers F.Cu B.Cu) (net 17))
 (segment (start 35.56 17.78) (end 35.56 22.86) (width 0.889) (layer B.Cu) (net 18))
 (segment (start 55.88 27.94) (end 53.34 27.94) (width 0.889) (layer B.Cu) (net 18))
 (segment (start 53.34 27.94) (end 53.34 20.32) (width 0.889) (layer F.Cu) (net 18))
 (segment (start 43.18 12.7) (end 48.26 12.7) (width 0.889) (layer F.Cu) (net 18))
 (segment (start 53.34 17.78) (end 53.34 20.32) (width 0.889) (layer B.Cu) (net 18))
 (segment (start 48.26 12.7) (end 53.34 17.78) (width 0.889) (layer B.Cu) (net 18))
 (via (at 53.34 20.32) (size 1.778) (drill 0.889) (layers F.Cu B.Cu) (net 18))
 (via (at 53.34 27.94) (size 1.778) (drill 0.889) (layers F.Cu B.Cu) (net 18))
 (via (at 43.18 12.7) (size 1.778) (drill 0.889) (layers F.Cu B.Cu) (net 18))
 (via (at 48.26 12.7) (size 1.778) (drill 0.889) (layers F.Cu B.Cu) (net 18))
 (segment (start 35.56 15.24) (end 35.56 17.78) (width 0.889) (layer B.Cu) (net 18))
 (segment (start 43.18 12.7) (end 35.56 12.7) (width 0.889) (layer B.Cu) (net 18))
 (segment (start 35.56 12.7) (end 35.56 15.24) (width 0.889) (layer B.Cu) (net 18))
 (segment (start 53.34 39.23137) (end 53.34 38.1) (width 0.889) (layer B.Cu) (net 23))
 (segment (start 52.464869 40.106501) (end 53.34 39.23137) (width 0.889) (layer B.Cu) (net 23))
 (segment (start 44.31137 45.72) (end 49.924869 40.106501) (width 0.889) (layer B.Cu) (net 23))
 (segment (start 49.924869 40.106501) (end 52.464869 40.106501) (width 0.889) (layer B.Cu) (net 23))
 (segment (start 43.18 45.72) (end 44.31137 45.72) (width 0.889) (layer B.Cu) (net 23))
 (segment (start 10.24382 20.23618) (end 7.62 22.86) (width 0.889) (layer B.Cu) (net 8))
 (segment (start 10.24382 17.78) (end 10.24382 20.23618) (width 0.889) (layer B.Cu) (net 8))
 (segment (start 34.42863 43.18) (end 35.56 43.18) (width 0.889) (layer B.Cu) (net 31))
 (segment (start 33.02 44.58863) (end 34.42863 43.18) (width 0.889) (layer B.Cu) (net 31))
 (segment (start 33.02 45.72) (end 33.02 44.58863) (width 0.889) (layer B.Cu) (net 31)))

